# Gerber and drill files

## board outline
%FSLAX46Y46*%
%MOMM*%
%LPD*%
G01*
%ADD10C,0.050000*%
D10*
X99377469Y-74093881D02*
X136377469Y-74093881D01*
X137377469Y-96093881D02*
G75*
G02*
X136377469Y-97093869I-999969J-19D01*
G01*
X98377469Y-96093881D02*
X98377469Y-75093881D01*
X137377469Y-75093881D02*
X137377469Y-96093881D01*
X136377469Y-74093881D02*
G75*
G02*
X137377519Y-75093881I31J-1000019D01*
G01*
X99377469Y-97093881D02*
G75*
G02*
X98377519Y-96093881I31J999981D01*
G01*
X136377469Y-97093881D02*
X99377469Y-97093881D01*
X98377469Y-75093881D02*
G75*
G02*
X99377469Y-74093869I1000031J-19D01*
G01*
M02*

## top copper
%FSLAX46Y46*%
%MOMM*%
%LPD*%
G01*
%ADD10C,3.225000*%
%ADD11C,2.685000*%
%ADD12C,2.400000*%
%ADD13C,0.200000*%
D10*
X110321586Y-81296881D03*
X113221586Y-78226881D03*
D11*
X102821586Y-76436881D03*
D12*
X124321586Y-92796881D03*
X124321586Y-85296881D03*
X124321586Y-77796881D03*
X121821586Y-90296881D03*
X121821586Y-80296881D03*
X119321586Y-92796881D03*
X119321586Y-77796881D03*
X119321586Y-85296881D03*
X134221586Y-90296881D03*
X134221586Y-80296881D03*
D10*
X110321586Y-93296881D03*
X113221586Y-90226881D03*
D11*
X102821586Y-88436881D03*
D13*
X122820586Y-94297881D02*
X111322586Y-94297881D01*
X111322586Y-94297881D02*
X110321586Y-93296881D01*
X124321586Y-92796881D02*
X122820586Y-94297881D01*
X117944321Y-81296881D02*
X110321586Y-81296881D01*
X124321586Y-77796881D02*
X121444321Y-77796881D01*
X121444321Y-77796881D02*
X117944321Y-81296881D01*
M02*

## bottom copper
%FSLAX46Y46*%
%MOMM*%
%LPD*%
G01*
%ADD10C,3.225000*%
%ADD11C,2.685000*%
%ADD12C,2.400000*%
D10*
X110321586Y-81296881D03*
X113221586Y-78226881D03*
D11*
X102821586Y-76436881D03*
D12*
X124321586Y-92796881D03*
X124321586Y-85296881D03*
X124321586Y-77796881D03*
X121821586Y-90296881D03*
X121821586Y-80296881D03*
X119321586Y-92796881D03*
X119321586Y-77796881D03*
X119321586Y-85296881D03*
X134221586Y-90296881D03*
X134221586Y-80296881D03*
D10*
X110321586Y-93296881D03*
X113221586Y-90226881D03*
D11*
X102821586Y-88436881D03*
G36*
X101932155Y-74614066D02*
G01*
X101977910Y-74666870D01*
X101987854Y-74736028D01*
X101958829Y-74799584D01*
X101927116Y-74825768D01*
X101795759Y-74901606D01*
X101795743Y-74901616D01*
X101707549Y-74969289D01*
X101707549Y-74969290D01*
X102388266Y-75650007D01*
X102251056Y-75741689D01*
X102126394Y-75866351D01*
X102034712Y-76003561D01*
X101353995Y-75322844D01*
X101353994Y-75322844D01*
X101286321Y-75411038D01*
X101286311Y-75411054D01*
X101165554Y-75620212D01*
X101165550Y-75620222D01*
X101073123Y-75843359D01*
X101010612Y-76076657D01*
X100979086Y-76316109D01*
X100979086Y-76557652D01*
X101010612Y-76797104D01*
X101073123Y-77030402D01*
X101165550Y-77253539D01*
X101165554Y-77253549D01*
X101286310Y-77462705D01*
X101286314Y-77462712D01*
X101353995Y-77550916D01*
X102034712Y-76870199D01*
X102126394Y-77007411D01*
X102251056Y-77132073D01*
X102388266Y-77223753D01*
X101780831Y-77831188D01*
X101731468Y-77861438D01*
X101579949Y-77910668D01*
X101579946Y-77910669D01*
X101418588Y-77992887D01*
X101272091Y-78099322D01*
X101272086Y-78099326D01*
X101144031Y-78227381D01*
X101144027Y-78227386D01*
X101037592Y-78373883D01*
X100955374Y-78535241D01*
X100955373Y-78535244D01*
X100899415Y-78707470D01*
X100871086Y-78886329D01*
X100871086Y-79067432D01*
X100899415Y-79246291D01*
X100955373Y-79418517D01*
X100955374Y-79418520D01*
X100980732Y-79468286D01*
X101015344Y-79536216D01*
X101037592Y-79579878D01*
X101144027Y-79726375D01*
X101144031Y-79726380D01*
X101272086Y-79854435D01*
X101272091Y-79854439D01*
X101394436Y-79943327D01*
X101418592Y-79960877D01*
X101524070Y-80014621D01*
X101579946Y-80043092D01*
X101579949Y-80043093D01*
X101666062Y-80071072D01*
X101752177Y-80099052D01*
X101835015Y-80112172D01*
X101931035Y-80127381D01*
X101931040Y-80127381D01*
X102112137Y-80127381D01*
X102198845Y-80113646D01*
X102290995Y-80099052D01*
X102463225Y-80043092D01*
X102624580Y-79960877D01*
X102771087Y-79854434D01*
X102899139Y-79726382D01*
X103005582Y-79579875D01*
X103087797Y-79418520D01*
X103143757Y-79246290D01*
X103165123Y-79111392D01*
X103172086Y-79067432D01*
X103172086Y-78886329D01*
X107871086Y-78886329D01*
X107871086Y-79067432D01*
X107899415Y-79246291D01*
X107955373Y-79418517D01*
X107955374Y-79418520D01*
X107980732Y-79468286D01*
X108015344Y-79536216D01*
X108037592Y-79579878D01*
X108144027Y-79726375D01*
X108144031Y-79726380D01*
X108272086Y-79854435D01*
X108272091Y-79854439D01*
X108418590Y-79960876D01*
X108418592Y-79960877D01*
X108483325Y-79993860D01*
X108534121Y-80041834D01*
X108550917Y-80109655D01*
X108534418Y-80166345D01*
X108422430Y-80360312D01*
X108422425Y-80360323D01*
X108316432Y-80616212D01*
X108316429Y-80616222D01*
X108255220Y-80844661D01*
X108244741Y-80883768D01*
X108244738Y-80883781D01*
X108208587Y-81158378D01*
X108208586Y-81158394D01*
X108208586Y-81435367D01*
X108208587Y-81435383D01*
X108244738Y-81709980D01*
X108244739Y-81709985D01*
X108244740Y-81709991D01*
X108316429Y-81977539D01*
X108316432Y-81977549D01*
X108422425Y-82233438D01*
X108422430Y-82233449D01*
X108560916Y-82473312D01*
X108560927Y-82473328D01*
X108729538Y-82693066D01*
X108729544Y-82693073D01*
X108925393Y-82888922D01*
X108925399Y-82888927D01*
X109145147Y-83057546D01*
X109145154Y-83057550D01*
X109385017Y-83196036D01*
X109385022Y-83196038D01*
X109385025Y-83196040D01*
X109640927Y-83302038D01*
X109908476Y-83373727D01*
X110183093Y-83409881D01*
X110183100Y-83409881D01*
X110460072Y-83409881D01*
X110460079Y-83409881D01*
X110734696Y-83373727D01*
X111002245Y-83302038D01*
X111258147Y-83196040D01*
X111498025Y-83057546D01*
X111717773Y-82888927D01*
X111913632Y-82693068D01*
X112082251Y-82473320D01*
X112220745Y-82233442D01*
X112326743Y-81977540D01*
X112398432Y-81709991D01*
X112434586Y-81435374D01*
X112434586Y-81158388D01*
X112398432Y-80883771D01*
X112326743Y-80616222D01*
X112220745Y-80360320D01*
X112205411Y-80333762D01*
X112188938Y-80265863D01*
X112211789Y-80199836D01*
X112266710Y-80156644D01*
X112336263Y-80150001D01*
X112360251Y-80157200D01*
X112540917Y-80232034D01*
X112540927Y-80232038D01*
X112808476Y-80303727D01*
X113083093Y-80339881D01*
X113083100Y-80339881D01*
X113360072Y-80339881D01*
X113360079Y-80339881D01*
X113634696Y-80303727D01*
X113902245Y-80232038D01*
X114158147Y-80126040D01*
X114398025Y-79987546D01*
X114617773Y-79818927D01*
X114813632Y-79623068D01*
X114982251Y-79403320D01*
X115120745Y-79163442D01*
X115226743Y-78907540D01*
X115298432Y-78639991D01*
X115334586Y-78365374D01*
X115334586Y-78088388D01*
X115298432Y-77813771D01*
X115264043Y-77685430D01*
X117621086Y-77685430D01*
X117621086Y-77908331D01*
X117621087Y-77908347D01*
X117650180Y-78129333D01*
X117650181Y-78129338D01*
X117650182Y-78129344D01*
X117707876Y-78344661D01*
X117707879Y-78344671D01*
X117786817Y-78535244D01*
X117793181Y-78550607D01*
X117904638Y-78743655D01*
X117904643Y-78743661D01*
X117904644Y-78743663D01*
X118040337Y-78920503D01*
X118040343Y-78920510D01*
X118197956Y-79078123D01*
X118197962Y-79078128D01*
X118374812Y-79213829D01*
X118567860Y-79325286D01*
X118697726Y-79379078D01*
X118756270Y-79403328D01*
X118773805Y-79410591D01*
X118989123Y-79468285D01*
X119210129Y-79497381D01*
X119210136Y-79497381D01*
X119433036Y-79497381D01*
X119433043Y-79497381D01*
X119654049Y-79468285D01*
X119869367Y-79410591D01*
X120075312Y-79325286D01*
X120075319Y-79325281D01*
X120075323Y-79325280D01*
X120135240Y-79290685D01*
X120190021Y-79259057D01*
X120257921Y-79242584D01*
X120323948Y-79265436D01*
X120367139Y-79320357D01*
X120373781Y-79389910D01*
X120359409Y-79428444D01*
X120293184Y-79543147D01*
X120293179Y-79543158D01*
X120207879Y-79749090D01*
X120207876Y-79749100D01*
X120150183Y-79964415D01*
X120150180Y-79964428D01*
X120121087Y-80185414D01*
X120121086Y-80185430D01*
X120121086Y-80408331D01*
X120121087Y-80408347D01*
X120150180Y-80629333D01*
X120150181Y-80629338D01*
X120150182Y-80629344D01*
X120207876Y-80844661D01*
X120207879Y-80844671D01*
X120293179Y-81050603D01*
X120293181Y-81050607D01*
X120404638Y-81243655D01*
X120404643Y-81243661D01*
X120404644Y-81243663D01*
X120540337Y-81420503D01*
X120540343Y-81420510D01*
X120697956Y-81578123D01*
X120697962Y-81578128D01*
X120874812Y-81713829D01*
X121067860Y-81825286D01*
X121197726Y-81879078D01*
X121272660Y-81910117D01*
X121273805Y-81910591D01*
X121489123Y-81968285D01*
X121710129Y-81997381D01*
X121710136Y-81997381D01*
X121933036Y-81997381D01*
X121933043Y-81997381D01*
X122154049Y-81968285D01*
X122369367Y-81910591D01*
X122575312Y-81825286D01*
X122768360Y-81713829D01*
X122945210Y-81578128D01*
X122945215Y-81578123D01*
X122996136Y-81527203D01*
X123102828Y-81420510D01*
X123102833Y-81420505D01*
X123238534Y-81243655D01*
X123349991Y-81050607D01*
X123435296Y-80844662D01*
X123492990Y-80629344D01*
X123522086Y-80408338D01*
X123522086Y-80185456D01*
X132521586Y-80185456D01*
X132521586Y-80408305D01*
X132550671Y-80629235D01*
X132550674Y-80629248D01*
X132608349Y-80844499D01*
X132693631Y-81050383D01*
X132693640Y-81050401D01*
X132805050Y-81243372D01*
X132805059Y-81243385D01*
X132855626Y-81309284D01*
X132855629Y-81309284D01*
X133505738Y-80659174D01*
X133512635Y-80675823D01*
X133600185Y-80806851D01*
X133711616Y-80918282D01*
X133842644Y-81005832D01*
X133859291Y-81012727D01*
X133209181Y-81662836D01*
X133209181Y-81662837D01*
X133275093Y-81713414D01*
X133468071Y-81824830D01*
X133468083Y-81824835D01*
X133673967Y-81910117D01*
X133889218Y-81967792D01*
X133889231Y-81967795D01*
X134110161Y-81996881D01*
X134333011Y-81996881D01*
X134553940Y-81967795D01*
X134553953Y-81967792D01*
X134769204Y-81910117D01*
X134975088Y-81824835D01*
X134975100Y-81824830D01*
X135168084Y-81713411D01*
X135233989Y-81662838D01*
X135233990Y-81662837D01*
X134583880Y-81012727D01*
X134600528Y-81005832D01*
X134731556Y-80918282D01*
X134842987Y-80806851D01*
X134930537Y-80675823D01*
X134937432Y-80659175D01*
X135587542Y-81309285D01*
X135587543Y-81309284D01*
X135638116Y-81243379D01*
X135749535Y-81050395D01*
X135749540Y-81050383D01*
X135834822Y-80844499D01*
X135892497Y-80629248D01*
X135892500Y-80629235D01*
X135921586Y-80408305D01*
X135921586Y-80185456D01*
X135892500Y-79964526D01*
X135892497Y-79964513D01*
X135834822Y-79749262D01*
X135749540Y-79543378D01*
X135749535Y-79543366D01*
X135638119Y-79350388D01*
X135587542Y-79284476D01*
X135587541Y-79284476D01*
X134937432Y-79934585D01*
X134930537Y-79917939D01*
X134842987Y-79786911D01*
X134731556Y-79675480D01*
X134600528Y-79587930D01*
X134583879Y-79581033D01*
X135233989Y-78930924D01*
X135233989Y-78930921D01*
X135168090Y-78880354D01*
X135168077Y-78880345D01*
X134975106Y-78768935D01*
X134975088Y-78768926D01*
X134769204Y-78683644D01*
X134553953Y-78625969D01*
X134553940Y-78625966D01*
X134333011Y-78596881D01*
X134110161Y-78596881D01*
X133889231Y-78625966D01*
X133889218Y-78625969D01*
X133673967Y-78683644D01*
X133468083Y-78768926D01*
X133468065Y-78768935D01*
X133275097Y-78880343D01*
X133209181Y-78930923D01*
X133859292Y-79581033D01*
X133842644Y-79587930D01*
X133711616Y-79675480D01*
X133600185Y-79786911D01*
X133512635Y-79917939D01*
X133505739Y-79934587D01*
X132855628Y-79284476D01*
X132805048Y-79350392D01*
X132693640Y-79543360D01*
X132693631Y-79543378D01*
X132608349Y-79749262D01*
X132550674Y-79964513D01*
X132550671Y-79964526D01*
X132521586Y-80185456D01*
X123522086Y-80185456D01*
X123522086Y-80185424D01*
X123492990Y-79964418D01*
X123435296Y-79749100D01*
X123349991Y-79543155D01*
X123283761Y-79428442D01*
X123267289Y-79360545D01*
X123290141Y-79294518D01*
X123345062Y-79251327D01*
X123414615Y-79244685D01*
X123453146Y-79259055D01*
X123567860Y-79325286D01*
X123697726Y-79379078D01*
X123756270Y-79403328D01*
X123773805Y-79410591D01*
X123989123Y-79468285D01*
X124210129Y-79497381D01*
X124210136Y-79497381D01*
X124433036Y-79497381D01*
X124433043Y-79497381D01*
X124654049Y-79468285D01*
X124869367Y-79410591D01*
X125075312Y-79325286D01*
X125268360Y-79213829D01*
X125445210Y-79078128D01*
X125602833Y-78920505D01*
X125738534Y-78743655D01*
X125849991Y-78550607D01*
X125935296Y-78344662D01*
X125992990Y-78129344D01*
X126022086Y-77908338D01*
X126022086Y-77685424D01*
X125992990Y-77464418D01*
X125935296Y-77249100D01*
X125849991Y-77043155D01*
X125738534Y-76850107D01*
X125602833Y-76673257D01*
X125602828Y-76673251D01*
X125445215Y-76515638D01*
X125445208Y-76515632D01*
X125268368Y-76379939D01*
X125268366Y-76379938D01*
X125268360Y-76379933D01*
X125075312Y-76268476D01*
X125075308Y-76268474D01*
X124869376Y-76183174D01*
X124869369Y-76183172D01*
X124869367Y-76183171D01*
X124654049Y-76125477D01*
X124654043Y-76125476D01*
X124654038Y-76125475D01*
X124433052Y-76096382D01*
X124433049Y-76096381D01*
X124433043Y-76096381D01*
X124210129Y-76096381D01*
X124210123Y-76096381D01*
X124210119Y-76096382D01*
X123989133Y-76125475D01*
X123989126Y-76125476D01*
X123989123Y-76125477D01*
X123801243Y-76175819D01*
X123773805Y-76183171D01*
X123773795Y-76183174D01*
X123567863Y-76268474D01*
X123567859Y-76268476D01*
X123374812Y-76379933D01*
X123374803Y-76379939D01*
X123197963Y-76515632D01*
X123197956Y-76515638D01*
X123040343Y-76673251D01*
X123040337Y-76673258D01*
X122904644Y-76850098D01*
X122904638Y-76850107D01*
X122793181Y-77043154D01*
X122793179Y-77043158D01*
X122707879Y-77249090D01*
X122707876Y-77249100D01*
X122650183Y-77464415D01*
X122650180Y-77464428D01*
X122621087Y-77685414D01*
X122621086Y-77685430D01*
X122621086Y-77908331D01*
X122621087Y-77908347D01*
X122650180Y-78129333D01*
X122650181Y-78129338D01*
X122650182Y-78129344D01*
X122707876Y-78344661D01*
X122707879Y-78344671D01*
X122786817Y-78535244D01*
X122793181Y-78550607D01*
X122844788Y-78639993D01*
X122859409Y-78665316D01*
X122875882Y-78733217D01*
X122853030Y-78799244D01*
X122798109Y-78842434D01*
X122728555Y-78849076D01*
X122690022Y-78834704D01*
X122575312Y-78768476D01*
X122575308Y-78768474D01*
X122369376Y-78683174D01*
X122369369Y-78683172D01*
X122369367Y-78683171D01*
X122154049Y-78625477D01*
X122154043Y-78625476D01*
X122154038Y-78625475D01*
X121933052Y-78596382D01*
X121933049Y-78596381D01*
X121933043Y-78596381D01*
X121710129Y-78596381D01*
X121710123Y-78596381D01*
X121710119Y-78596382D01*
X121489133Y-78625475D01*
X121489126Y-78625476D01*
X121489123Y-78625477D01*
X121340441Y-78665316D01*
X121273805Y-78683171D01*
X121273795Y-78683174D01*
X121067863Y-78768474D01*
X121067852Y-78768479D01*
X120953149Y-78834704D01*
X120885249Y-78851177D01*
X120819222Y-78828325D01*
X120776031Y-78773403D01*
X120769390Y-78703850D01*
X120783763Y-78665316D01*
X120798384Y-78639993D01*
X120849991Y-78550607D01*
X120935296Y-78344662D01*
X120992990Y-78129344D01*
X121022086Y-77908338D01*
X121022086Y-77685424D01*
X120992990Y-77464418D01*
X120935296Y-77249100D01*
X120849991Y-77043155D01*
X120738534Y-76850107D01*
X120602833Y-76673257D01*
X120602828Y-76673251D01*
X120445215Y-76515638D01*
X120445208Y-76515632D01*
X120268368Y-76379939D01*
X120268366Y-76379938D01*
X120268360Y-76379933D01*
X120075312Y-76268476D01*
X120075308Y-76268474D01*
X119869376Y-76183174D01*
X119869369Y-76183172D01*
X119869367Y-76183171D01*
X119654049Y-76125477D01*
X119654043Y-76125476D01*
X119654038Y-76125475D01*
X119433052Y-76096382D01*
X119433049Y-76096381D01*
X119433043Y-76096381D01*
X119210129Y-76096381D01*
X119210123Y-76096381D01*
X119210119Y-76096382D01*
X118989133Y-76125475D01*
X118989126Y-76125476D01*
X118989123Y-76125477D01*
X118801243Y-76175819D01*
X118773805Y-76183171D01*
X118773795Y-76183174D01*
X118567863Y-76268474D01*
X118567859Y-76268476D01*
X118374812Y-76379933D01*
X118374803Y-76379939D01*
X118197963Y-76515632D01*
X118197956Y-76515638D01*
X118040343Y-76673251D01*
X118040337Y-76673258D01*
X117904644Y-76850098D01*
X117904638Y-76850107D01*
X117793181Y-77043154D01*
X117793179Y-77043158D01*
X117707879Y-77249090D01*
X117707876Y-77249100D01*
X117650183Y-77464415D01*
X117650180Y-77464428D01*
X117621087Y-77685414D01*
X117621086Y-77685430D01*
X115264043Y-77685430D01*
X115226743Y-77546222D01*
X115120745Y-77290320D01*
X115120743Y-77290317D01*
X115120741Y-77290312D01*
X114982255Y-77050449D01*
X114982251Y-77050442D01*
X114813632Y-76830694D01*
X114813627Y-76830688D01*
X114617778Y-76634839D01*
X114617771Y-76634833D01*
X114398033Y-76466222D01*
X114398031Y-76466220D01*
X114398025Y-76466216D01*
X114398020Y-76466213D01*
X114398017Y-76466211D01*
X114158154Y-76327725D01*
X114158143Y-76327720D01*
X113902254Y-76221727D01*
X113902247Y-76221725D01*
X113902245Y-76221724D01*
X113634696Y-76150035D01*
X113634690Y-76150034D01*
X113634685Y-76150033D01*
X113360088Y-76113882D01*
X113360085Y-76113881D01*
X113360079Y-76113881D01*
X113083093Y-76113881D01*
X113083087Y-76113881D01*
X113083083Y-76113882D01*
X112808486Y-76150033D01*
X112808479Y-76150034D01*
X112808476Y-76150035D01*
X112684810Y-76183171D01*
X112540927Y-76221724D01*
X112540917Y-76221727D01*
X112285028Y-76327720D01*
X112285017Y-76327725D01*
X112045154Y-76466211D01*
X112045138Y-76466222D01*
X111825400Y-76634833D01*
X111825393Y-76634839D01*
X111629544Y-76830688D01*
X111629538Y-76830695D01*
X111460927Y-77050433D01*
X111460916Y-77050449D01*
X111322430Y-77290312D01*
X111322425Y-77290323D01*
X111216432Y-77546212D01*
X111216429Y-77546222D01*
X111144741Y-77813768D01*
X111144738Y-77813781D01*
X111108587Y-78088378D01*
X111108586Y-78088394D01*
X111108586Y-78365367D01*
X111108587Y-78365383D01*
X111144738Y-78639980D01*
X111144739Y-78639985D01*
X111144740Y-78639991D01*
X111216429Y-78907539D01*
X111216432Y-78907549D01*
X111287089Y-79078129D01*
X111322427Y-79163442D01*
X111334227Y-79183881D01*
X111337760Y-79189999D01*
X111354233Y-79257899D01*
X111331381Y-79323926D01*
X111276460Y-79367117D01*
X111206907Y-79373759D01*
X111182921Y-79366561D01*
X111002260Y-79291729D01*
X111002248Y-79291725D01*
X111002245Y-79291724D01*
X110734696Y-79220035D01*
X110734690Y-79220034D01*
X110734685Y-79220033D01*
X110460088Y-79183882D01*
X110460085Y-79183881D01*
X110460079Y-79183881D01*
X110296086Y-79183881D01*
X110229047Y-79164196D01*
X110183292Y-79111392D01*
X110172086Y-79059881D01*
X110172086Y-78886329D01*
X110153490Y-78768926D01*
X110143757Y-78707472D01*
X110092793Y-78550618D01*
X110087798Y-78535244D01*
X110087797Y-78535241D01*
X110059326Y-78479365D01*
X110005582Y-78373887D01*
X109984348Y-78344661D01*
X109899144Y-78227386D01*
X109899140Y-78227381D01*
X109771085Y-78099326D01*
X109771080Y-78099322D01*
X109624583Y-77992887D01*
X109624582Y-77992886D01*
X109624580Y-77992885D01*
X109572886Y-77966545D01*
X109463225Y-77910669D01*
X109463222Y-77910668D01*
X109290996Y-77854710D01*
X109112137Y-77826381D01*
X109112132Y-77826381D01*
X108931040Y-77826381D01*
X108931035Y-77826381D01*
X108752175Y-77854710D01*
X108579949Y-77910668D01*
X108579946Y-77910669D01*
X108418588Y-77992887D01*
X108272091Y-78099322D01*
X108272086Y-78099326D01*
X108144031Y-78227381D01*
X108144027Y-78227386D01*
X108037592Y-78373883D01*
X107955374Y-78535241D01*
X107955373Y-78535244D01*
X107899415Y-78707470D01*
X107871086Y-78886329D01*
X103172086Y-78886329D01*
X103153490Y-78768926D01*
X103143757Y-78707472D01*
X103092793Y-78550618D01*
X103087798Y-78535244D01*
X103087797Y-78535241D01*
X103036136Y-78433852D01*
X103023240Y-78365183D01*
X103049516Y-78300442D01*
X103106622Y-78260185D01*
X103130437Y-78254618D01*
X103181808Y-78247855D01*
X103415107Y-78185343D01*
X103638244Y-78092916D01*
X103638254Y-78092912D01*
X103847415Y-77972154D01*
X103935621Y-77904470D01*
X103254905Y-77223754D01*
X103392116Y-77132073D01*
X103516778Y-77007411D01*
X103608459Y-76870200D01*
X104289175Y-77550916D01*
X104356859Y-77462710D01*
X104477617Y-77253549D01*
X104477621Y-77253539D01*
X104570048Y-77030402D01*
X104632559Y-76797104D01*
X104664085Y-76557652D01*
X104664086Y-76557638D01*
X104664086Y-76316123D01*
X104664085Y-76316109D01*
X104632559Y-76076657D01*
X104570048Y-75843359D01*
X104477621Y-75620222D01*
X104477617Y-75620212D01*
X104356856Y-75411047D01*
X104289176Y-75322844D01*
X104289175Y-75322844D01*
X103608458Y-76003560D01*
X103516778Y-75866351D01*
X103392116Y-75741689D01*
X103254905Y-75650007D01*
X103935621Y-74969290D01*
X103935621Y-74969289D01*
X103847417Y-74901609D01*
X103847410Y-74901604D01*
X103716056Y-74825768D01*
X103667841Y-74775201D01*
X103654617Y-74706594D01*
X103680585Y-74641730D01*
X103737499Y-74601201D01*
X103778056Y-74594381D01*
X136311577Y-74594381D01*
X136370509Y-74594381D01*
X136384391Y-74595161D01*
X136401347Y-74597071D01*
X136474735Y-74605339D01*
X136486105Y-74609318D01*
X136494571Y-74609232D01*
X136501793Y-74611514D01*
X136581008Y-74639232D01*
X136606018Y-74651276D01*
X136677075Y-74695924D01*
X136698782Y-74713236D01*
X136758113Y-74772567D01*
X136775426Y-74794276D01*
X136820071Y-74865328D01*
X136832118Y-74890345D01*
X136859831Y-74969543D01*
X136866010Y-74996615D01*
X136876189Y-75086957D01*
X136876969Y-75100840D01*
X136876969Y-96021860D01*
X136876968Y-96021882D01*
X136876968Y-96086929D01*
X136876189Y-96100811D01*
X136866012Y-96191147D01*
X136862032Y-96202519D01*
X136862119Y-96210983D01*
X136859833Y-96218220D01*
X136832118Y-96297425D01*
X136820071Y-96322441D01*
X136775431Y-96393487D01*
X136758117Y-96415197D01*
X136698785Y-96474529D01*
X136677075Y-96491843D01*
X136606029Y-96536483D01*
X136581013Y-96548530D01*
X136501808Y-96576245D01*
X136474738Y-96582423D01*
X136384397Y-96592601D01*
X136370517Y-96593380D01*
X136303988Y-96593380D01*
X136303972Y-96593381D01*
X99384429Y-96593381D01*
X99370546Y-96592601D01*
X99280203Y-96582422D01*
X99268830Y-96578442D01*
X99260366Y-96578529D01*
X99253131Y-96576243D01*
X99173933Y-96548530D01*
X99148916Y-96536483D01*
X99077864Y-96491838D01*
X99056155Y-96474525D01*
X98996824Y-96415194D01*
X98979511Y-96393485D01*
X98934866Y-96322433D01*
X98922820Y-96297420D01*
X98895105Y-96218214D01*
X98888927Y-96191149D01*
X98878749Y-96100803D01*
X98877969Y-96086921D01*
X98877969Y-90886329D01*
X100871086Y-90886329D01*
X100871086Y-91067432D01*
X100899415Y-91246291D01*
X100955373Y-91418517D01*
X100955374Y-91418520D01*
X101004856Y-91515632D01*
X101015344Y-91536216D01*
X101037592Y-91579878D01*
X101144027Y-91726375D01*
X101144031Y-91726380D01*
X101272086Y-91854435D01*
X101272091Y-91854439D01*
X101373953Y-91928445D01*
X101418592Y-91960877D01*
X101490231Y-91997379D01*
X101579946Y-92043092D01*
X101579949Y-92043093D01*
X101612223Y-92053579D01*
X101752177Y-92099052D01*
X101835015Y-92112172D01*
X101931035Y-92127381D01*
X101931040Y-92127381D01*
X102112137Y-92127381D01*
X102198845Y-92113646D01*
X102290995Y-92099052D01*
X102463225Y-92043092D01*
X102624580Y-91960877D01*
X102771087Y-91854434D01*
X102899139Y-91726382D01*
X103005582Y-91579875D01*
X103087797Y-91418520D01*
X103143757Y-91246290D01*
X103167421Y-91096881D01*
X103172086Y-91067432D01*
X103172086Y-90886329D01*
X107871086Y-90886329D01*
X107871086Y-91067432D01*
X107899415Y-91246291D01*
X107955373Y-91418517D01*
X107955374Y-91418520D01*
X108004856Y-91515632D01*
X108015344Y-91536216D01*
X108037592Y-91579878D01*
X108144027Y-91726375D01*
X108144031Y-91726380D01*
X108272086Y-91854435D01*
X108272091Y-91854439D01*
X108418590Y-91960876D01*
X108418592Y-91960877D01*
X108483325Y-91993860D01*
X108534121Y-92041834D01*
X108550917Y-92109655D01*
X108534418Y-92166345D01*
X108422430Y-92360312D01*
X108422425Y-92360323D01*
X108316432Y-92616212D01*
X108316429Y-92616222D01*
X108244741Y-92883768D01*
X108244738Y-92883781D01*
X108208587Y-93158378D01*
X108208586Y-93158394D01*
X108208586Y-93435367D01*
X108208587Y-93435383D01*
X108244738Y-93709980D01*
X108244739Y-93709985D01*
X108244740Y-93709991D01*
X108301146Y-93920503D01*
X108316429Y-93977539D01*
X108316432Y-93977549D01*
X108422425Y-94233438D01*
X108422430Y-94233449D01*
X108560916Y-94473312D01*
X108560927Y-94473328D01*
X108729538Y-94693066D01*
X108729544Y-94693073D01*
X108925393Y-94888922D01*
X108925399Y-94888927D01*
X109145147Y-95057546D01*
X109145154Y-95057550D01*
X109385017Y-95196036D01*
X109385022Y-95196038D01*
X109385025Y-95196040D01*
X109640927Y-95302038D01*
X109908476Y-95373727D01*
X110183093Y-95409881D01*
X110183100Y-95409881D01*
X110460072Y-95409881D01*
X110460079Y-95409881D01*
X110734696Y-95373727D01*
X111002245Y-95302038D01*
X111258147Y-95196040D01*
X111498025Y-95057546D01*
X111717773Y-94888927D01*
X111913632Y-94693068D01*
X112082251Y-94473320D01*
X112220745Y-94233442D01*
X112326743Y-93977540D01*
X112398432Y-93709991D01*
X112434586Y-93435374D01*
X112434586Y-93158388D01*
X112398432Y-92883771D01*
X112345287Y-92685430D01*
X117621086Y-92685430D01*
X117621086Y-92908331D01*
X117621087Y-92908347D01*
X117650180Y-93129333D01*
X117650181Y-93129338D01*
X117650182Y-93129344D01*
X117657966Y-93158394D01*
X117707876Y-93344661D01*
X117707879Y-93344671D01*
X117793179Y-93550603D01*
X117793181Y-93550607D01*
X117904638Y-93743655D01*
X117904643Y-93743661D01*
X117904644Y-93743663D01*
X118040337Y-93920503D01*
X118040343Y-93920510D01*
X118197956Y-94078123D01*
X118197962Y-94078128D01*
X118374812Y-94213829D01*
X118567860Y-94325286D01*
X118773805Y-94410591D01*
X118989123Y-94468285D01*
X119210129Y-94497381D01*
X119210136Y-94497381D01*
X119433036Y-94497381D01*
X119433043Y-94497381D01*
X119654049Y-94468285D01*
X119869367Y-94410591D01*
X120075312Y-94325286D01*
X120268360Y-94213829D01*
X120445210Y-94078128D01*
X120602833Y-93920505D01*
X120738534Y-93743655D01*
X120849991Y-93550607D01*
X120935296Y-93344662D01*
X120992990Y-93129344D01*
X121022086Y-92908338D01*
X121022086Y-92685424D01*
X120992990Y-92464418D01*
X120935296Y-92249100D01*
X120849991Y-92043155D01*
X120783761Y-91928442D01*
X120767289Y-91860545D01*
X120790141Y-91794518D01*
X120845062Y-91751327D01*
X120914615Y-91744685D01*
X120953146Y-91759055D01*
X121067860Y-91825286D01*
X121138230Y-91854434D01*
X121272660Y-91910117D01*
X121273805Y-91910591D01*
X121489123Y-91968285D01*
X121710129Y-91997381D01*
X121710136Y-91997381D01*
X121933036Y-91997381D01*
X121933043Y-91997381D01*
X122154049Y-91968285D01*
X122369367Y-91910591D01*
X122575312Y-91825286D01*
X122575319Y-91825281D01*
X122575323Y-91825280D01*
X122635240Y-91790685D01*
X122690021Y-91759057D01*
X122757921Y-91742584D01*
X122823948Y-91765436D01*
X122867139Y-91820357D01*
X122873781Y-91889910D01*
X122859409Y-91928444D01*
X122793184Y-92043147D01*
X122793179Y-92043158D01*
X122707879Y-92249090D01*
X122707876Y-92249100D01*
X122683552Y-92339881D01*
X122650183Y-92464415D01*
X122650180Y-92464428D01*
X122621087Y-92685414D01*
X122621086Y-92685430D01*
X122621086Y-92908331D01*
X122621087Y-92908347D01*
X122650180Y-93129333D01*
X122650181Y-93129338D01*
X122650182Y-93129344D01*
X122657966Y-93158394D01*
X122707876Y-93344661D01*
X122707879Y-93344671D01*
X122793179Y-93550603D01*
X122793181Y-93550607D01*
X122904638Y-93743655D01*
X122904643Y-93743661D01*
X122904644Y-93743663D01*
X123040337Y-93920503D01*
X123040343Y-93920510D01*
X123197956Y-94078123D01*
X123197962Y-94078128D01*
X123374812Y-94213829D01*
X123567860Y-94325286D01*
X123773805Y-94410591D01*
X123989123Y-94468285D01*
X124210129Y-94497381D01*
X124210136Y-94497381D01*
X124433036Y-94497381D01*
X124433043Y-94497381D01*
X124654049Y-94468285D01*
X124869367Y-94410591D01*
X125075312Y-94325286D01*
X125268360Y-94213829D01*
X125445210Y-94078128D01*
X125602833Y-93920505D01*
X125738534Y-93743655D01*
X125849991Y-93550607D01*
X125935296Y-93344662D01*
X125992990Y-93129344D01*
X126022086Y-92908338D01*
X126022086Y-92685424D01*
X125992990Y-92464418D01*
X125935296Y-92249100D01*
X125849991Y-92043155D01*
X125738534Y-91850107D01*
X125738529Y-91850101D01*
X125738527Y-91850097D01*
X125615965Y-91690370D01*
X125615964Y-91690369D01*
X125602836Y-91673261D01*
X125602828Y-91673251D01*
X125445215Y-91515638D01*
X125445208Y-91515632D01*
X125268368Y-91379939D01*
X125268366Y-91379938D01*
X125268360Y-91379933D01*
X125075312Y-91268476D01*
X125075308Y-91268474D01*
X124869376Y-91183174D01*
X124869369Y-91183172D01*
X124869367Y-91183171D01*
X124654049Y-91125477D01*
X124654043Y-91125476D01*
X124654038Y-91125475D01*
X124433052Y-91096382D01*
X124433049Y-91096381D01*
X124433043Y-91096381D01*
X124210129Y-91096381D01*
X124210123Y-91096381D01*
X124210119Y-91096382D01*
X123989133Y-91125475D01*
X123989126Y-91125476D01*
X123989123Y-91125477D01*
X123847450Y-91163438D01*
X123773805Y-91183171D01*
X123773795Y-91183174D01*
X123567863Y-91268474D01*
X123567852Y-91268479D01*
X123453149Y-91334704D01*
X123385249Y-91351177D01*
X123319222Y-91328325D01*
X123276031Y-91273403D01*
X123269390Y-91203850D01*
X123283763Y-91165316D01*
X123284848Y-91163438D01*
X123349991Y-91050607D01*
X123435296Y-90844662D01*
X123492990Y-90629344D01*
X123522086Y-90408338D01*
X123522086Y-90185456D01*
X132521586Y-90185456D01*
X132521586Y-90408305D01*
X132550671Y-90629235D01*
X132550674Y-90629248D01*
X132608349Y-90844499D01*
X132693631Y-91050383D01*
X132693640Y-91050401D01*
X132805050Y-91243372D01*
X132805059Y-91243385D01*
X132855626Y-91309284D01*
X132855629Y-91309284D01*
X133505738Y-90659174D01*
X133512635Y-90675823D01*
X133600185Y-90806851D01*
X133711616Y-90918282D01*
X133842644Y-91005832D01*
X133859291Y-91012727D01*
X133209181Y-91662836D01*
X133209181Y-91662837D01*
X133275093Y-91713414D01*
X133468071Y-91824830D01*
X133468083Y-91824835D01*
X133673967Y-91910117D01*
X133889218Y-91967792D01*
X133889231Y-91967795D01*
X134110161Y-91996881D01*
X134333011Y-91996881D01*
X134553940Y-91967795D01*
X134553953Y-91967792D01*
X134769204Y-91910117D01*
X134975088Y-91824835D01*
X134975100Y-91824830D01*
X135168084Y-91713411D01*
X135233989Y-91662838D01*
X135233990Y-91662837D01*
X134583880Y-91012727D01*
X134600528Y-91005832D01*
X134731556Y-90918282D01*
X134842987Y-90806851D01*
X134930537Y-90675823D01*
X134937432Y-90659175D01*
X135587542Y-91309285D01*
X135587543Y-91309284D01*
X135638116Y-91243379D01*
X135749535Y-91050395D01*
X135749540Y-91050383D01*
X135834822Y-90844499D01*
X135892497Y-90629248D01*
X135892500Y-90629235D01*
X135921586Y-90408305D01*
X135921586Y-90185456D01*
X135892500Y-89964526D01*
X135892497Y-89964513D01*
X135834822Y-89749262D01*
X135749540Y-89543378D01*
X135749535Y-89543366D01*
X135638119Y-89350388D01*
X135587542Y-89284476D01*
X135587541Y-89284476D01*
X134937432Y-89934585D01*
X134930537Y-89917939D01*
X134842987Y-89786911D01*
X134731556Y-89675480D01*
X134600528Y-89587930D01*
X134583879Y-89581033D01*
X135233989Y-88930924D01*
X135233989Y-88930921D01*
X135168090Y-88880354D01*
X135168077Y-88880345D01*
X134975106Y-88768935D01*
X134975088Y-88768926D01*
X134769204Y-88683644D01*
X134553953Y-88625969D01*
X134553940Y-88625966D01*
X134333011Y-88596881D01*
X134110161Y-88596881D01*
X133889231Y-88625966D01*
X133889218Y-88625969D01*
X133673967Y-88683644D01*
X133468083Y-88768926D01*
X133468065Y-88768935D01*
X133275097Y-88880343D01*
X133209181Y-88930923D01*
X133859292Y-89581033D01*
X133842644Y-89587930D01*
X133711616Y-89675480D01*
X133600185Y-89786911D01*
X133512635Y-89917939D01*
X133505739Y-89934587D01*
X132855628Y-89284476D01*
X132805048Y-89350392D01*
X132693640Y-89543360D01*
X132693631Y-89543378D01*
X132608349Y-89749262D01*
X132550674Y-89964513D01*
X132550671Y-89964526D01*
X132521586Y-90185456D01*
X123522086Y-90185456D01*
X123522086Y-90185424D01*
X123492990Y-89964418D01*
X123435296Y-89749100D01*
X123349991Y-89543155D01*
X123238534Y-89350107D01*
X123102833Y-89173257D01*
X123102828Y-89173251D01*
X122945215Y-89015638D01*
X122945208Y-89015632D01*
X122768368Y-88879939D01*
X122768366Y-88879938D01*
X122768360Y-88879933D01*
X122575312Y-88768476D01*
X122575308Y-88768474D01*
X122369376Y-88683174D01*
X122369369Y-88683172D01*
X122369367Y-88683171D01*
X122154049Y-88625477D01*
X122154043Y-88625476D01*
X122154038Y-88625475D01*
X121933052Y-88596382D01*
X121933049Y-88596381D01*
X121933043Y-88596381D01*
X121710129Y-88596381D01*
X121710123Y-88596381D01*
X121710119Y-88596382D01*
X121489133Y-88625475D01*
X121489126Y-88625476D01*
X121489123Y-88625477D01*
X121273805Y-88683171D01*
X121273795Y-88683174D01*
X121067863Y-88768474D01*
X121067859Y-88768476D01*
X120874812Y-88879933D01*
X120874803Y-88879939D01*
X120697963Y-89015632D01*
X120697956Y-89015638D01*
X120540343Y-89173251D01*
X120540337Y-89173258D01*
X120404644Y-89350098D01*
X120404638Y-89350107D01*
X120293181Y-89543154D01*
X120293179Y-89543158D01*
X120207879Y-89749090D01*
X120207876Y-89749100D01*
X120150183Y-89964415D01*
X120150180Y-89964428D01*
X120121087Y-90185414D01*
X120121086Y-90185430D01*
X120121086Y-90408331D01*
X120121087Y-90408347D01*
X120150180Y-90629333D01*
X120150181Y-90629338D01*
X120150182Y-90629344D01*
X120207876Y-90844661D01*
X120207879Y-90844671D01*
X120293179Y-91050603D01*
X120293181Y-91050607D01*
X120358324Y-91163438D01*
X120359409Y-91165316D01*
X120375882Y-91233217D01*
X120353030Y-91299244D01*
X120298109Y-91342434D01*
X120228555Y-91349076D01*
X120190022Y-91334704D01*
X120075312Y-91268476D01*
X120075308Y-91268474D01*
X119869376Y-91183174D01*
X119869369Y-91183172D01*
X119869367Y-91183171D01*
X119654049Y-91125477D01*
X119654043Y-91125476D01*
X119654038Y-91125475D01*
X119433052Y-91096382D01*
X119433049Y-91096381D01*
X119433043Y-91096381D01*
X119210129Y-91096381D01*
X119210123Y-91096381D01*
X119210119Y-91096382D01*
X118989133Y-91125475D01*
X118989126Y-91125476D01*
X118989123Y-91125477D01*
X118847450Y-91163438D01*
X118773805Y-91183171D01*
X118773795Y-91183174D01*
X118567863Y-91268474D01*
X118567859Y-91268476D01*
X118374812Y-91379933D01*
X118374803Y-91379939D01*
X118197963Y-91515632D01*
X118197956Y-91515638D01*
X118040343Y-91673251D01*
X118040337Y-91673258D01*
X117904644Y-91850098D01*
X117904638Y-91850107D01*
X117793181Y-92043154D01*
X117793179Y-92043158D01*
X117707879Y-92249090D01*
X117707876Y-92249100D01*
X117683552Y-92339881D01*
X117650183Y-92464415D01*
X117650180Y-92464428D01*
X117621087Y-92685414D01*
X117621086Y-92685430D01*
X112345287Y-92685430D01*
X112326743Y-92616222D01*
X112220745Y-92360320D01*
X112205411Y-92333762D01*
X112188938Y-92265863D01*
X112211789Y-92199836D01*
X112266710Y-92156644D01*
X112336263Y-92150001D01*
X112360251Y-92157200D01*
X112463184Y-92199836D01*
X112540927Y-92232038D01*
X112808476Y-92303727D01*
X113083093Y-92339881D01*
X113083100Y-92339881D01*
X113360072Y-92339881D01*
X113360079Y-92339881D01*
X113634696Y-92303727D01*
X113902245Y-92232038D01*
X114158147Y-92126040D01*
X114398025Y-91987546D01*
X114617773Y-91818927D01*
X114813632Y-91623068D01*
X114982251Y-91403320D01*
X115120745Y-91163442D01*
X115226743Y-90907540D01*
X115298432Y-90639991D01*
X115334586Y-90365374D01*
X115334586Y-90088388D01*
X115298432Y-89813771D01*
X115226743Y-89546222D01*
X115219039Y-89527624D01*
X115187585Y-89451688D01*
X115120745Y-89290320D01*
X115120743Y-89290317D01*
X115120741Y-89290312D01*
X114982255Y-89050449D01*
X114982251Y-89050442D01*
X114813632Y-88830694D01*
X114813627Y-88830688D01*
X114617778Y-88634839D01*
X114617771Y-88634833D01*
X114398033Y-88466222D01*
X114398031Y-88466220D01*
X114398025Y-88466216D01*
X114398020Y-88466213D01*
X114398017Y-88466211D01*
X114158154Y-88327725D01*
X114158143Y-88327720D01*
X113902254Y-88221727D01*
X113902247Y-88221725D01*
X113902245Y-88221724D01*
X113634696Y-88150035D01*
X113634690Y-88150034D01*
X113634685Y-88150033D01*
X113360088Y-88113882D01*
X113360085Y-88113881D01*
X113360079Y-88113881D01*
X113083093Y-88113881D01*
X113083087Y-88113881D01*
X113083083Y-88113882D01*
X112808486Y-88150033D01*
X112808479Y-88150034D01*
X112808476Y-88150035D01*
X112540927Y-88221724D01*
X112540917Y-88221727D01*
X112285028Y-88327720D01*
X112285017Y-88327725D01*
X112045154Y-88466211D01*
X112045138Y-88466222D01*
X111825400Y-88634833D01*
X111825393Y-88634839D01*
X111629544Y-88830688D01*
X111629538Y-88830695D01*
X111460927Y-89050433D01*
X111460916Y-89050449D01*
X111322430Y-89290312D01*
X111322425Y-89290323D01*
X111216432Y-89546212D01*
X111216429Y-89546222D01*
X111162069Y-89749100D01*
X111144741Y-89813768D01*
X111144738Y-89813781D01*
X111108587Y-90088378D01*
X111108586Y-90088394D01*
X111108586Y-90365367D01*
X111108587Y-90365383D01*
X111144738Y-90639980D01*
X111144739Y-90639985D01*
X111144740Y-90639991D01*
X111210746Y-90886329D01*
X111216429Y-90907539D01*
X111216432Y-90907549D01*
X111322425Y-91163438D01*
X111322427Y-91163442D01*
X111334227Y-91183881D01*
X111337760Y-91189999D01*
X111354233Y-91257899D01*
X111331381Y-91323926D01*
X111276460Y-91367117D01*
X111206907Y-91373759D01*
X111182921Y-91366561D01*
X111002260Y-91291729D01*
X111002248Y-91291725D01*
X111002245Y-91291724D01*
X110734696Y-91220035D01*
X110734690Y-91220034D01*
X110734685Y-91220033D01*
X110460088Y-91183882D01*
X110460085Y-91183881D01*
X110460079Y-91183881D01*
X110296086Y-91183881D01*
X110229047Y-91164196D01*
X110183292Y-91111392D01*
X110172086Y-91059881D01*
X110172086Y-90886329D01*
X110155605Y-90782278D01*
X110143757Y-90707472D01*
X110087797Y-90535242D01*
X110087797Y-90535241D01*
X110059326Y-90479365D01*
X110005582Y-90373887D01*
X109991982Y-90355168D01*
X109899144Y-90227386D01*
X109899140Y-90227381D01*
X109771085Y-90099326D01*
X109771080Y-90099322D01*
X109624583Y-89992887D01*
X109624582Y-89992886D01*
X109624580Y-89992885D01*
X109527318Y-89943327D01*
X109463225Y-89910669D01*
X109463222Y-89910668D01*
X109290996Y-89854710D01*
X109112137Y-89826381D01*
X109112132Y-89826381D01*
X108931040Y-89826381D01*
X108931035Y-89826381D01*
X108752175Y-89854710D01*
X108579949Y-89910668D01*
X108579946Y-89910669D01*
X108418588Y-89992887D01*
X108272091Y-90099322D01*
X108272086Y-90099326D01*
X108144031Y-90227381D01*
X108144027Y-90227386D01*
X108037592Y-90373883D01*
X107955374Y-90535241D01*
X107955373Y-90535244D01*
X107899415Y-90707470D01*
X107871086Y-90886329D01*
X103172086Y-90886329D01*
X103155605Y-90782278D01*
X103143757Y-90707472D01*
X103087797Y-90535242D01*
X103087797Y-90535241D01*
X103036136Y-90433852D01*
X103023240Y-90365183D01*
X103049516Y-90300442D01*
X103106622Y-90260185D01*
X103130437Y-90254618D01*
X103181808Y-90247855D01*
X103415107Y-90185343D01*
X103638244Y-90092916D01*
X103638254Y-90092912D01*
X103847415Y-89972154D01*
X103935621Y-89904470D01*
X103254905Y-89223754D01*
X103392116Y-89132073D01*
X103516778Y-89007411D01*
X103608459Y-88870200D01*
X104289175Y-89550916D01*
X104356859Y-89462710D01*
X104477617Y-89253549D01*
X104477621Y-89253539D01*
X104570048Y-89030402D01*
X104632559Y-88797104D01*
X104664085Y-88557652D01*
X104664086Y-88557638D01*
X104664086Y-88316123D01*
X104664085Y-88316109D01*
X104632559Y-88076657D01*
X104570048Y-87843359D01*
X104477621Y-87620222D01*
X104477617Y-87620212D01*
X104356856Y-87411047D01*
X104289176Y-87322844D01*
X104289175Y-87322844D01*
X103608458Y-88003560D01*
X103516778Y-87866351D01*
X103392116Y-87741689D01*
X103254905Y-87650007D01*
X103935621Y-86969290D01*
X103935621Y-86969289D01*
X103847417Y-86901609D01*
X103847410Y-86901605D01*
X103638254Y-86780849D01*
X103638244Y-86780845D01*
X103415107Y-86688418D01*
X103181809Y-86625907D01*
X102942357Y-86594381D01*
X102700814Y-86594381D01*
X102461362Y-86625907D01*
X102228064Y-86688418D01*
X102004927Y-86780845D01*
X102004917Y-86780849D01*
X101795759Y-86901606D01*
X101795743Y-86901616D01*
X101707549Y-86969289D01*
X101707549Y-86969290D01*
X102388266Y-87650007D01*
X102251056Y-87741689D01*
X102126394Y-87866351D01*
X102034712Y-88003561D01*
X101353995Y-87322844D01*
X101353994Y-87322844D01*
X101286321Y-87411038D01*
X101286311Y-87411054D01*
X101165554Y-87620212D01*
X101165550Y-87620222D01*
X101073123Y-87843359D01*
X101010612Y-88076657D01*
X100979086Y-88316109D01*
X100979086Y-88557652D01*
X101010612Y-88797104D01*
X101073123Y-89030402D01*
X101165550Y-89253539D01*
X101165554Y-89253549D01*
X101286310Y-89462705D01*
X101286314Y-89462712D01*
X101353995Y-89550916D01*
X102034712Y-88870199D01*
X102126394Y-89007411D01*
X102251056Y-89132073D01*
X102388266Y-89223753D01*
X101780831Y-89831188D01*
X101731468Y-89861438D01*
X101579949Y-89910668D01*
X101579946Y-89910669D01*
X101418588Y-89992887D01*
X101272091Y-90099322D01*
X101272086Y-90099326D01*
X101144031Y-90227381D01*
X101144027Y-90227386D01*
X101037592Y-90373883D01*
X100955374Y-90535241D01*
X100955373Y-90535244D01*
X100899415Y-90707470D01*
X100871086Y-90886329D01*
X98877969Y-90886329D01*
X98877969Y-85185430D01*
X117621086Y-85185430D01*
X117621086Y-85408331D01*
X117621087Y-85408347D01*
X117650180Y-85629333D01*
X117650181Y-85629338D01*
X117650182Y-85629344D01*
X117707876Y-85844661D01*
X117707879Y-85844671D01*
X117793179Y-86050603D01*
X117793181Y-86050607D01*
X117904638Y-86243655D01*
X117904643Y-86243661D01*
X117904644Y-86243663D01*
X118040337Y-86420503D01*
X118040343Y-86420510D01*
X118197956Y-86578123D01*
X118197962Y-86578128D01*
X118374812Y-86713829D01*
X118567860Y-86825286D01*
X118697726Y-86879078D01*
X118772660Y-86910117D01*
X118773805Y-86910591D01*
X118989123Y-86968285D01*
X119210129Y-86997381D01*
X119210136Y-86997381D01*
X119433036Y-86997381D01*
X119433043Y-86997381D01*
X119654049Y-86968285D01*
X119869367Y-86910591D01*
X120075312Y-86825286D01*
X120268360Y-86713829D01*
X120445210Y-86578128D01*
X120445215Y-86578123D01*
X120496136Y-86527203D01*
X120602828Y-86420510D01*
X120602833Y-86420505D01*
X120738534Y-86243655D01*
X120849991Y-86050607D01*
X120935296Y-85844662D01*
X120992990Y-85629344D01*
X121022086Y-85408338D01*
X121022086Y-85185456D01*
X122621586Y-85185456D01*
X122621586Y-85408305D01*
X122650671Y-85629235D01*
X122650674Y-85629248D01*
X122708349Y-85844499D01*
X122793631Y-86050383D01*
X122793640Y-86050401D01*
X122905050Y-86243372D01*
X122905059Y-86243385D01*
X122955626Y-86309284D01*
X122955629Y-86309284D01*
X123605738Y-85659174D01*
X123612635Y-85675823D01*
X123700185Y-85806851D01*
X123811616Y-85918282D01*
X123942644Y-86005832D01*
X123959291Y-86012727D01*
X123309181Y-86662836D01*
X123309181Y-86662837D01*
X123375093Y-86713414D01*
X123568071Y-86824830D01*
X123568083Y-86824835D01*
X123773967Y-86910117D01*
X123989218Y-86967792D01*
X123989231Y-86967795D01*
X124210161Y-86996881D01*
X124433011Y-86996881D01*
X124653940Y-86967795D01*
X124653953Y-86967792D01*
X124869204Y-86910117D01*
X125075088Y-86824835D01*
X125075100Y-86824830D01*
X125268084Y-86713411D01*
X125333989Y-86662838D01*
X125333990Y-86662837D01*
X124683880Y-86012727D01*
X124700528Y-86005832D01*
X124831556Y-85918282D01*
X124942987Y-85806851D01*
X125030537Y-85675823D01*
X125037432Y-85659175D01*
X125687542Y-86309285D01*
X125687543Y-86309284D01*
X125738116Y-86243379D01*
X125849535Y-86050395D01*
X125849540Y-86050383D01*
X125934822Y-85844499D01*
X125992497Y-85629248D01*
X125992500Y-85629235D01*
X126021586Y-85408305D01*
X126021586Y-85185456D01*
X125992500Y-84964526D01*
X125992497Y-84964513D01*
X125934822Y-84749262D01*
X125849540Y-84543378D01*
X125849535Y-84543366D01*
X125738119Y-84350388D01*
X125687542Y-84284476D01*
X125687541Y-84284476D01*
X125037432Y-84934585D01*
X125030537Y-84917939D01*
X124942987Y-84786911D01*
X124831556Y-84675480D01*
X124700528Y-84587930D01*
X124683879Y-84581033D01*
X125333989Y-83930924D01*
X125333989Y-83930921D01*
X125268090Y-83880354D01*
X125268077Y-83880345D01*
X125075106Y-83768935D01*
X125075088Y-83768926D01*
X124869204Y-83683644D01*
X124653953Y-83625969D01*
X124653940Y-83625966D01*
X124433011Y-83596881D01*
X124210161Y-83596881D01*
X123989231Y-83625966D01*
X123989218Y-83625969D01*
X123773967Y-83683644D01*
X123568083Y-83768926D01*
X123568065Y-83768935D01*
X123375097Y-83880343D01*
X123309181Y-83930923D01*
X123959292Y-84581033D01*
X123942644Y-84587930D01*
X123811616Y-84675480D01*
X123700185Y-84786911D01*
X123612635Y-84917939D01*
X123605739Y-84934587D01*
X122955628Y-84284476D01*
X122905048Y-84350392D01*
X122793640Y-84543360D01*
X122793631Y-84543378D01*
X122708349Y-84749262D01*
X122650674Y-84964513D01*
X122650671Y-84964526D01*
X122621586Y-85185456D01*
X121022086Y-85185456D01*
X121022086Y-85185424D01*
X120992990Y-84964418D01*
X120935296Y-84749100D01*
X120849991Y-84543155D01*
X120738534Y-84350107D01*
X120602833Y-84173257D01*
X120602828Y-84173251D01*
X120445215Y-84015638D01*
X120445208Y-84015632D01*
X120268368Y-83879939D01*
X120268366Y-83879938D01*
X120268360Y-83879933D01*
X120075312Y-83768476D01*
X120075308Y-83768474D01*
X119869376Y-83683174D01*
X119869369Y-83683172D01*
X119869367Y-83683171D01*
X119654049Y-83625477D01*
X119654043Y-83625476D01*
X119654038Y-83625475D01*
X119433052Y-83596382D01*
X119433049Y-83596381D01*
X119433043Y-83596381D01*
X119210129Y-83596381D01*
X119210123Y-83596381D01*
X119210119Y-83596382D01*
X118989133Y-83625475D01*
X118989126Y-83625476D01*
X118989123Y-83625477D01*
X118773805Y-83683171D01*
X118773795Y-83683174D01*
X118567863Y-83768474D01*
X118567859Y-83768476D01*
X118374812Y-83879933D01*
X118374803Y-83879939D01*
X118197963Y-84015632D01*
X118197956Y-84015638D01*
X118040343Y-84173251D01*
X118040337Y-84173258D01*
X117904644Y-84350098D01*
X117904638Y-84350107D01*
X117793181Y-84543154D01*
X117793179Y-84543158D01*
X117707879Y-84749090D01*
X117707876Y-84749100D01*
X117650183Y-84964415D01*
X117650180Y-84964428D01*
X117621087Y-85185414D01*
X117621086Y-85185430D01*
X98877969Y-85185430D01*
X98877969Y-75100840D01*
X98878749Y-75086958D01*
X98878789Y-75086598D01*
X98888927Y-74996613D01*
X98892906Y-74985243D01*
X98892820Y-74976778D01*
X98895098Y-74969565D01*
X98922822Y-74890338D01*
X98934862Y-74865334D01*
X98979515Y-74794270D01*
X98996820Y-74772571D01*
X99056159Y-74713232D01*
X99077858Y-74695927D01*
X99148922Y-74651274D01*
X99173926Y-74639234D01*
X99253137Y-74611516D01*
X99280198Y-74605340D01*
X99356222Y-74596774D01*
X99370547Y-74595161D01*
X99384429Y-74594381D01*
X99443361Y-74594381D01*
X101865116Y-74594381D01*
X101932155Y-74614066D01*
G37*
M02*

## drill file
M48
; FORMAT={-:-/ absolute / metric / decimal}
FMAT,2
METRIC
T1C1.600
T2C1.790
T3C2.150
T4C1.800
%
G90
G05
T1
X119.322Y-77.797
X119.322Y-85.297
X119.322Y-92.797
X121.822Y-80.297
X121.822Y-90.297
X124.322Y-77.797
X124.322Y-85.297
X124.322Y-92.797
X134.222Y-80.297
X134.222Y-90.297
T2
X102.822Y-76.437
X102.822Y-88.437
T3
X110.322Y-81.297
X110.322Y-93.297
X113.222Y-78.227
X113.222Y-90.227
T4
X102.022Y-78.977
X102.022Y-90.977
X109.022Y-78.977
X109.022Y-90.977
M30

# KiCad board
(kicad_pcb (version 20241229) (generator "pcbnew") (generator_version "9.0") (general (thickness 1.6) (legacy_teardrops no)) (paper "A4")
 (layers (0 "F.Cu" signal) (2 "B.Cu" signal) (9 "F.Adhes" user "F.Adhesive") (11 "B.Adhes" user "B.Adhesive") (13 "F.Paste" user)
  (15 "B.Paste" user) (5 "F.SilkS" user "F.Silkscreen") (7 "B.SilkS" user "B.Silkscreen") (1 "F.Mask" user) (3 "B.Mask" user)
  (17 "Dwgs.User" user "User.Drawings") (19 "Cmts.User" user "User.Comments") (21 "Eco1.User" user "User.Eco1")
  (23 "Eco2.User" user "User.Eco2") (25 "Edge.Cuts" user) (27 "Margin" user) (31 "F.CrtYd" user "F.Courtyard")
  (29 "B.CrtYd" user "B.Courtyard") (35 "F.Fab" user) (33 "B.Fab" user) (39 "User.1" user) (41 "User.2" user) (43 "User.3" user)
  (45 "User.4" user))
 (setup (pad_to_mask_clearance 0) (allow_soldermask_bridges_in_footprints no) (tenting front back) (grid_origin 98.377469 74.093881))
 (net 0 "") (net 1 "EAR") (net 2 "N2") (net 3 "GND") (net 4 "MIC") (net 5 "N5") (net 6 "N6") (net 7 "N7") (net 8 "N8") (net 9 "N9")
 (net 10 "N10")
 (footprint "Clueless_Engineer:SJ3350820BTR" (layer "F.Cu") (at 110.321586 81.296881)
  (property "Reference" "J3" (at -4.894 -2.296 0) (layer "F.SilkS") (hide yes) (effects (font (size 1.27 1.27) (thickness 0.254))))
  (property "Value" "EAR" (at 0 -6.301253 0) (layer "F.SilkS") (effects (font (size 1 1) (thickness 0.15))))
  (pad "" np_thru_hole circle (at -8.3 -2.32) (size 1.8 1.8) (drill 1.8) (layers "*.Cu" "*.Mask"))
  (pad "" np_thru_hole circle (at -1.3 -2.32) (size 1.8 1.8) (drill 1.8) (layers "*.Cu" "*.Mask"))
  (pad "2" thru_hole circle (at 0 0) (size 3.225 3.225) (drill 2.15) (layers "*.Cu" "*.Mask") (remove_unused_layers no) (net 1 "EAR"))
  (pad "3" thru_hole circle (at 2.9 -3.07) (size 3.225 3.225) (drill 2.15) (layers "*.Cu" "*.Mask") (remove_unused_layers no) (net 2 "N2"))
  (pad "5" thru_hole circle (at -7.5 -4.86) (size 2.685 2.685) (drill 1.79) (layers "*.Cu" "*.Mask") (remove_unused_layers no) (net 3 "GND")))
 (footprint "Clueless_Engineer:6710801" (layer "F.Cu") (at 124.321586 92.796881 -90)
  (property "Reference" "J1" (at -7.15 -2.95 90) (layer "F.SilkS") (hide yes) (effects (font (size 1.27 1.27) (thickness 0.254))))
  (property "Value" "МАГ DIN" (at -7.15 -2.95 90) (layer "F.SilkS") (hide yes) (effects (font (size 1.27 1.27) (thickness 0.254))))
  (pad "1" thru_hole circle (at 0 0 270) (size 2.4 2.4) (drill 1.6) (layers "*.Cu" "*.Mask") (remove_unused_layers no) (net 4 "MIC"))
  (pad "2" thru_hole circle (at -7.5 0 270) (size 2.4 2.4) (drill 1.6) (layers "*.Cu" "*.Mask") (remove_unused_layers no) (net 3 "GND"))
  (pad "3" thru_hole circle (at -15 0 270) (size 2.4 2.4) (drill 1.6) (layers "*.Cu" "*.Mask") (remove_unused_layers no) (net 1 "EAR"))
  (pad "4" thru_hole circle (at -2.5 2.5 270) (size 2.4 2.4) (drill 1.6) (layers "*.Cu" "*.Mask") (remove_unused_layers no) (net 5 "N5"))
  (pad "5" thru_hole circle (at -12.5 2.5 270) (size 2.4 2.4) (drill 1.6) (layers "*.Cu" "*.Mask") (remove_unused_layers no) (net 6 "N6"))
  (pad "6" thru_hole circle (at 0 5 270) (size 2.4 2.4) (drill 1.6) (layers "*.Cu" "*.Mask") (remove_unused_layers no) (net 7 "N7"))
  (pad "7" thru_hole circle (at -15 5 270) (size 2.4 2.4) (drill 1.6) (layers "*.Cu" "*.Mask") (remove_unused_layers no) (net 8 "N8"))
  (pad "8" thru_hole circle (at -7.5 5 270) (size 2.4 2.4) (drill 1.6) (layers "*.Cu" "*.Mask") (remove_unused_layers no) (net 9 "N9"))
  (pad "MH1" thru_hole circle (at -2.5 -9.9 270) (size 2.4 2.4) (drill 1.6) (layers "*.Cu" "*.Mask") (remove_unused_layers no) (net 3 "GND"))
  (pad "MH2" thru_hole circle (at -12.5 -9.9 270) (size 2.4 2.4) (drill 1.6) (layers "*.Cu" "*.Mask") (remove_unused_layers no)
   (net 3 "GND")))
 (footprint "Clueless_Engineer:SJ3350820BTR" (layer "F.Cu") (at 110.321586 93.296881)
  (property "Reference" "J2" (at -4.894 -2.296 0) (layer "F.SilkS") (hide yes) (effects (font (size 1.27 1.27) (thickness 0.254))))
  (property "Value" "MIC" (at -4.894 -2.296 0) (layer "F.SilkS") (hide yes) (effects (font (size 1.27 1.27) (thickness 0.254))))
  (pad "" np_thru_hole circle (at -8.3 -2.32) (size 1.8 1.8) (drill 1.8) (layers "*.Cu" "*.Mask"))
  (pad "" np_thru_hole circle (at -1.3 -2.32) (size 1.8 1.8) (drill 1.8) (layers "*.Cu" "*.Mask"))
  (pad "2" thru_hole circle (at 0 0) (size 3.225 3.225) (drill 2.15) (layers "*.Cu" "*.Mask") (remove_unused_layers no) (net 4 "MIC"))
  (pad "3" thru_hole circle (at 2.9 -3.07) (size 3.225 3.225) (drill 2.15) (layers "*.Cu" "*.Mask") (remove_unused_layers no) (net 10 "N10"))
  (pad "5" thru_hole circle (at -7.5 -4.86) (size 2.685 2.685) (drill 1.79) (layers "*.Cu" "*.Mask") (remove_unused_layers no) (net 3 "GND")))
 (gr_line (start 99.377469 74.093881) (end 136.377469 74.093881) (stroke (width 0.05) (type default)) (layer "Edge.Cuts"))
 (gr_arc (start 137.377469 96.093881) (mid 137.084581 96.800989) (end 136.377469 97.093881) (stroke (width 0.05) (type default))
  (layer "Edge.Cuts"))
 (gr_line (start 98.377469 96.093881) (end 98.377469 75.093881) (stroke (width 0.05) (type default)) (layer "Edge.Cuts"))
 (gr_line (start 137.377469 75.093881) (end 137.377469 96.093881) (stroke (width 0.05) (type default)) (layer "Edge.Cuts"))
 (gr_arc (start 136.377469 74.093881) (mid 137.084576 74.386774) (end 137.377469 75.093881) (stroke (width 0.05) (type default))
  (layer "Edge.Cuts"))
 (gr_arc (start 99.377469 97.093881) (mid 98.670362 96.800988) (end 98.377469 96.093881) (stroke (width 0.05) (type default))
  (layer "Edge.Cuts"))
 (gr_line (start 136.377469 97.093881) (end 99.377469 97.093881) (stroke (width 0.05) (type default)) (layer "Edge.Cuts"))
 (gr_arc (start 98.377469 75.093881) (mid 98.670362 74.386774) (end 99.377469 74.093881) (stroke (width 0.05) (type default))
  (layer "Edge.Cuts"))
 (segment (start 122.820586 94.297881) (end 111.322586 94.297881) (width 0.2) (layer "F.Cu") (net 4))
 (segment (start 111.322586 94.297881) (end 110.321586 93.296881) (width 0.2) (layer "F.Cu") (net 4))
 (segment (start 124.321586 92.796881) (end 122.820586 94.297881) (width 0.2) (layer "F.Cu") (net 4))
 (segment (start 117.944321 81.296881) (end 110.321586 81.296881) (width 0.2) (layer "F.Cu") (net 1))
 (segment (start 124.321586 77.796881) (end 121.444321 77.796881) (width 0.2) (layer "F.Cu") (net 1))
 (segment (start 121.444321 77.796881) (end 117.944321 81.296881) (width 0.2) (layer "F.Cu") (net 1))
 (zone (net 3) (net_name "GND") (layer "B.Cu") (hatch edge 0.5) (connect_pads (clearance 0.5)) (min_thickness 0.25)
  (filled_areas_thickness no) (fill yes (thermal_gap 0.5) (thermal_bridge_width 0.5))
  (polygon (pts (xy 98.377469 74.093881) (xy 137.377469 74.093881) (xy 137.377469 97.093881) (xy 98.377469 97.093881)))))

